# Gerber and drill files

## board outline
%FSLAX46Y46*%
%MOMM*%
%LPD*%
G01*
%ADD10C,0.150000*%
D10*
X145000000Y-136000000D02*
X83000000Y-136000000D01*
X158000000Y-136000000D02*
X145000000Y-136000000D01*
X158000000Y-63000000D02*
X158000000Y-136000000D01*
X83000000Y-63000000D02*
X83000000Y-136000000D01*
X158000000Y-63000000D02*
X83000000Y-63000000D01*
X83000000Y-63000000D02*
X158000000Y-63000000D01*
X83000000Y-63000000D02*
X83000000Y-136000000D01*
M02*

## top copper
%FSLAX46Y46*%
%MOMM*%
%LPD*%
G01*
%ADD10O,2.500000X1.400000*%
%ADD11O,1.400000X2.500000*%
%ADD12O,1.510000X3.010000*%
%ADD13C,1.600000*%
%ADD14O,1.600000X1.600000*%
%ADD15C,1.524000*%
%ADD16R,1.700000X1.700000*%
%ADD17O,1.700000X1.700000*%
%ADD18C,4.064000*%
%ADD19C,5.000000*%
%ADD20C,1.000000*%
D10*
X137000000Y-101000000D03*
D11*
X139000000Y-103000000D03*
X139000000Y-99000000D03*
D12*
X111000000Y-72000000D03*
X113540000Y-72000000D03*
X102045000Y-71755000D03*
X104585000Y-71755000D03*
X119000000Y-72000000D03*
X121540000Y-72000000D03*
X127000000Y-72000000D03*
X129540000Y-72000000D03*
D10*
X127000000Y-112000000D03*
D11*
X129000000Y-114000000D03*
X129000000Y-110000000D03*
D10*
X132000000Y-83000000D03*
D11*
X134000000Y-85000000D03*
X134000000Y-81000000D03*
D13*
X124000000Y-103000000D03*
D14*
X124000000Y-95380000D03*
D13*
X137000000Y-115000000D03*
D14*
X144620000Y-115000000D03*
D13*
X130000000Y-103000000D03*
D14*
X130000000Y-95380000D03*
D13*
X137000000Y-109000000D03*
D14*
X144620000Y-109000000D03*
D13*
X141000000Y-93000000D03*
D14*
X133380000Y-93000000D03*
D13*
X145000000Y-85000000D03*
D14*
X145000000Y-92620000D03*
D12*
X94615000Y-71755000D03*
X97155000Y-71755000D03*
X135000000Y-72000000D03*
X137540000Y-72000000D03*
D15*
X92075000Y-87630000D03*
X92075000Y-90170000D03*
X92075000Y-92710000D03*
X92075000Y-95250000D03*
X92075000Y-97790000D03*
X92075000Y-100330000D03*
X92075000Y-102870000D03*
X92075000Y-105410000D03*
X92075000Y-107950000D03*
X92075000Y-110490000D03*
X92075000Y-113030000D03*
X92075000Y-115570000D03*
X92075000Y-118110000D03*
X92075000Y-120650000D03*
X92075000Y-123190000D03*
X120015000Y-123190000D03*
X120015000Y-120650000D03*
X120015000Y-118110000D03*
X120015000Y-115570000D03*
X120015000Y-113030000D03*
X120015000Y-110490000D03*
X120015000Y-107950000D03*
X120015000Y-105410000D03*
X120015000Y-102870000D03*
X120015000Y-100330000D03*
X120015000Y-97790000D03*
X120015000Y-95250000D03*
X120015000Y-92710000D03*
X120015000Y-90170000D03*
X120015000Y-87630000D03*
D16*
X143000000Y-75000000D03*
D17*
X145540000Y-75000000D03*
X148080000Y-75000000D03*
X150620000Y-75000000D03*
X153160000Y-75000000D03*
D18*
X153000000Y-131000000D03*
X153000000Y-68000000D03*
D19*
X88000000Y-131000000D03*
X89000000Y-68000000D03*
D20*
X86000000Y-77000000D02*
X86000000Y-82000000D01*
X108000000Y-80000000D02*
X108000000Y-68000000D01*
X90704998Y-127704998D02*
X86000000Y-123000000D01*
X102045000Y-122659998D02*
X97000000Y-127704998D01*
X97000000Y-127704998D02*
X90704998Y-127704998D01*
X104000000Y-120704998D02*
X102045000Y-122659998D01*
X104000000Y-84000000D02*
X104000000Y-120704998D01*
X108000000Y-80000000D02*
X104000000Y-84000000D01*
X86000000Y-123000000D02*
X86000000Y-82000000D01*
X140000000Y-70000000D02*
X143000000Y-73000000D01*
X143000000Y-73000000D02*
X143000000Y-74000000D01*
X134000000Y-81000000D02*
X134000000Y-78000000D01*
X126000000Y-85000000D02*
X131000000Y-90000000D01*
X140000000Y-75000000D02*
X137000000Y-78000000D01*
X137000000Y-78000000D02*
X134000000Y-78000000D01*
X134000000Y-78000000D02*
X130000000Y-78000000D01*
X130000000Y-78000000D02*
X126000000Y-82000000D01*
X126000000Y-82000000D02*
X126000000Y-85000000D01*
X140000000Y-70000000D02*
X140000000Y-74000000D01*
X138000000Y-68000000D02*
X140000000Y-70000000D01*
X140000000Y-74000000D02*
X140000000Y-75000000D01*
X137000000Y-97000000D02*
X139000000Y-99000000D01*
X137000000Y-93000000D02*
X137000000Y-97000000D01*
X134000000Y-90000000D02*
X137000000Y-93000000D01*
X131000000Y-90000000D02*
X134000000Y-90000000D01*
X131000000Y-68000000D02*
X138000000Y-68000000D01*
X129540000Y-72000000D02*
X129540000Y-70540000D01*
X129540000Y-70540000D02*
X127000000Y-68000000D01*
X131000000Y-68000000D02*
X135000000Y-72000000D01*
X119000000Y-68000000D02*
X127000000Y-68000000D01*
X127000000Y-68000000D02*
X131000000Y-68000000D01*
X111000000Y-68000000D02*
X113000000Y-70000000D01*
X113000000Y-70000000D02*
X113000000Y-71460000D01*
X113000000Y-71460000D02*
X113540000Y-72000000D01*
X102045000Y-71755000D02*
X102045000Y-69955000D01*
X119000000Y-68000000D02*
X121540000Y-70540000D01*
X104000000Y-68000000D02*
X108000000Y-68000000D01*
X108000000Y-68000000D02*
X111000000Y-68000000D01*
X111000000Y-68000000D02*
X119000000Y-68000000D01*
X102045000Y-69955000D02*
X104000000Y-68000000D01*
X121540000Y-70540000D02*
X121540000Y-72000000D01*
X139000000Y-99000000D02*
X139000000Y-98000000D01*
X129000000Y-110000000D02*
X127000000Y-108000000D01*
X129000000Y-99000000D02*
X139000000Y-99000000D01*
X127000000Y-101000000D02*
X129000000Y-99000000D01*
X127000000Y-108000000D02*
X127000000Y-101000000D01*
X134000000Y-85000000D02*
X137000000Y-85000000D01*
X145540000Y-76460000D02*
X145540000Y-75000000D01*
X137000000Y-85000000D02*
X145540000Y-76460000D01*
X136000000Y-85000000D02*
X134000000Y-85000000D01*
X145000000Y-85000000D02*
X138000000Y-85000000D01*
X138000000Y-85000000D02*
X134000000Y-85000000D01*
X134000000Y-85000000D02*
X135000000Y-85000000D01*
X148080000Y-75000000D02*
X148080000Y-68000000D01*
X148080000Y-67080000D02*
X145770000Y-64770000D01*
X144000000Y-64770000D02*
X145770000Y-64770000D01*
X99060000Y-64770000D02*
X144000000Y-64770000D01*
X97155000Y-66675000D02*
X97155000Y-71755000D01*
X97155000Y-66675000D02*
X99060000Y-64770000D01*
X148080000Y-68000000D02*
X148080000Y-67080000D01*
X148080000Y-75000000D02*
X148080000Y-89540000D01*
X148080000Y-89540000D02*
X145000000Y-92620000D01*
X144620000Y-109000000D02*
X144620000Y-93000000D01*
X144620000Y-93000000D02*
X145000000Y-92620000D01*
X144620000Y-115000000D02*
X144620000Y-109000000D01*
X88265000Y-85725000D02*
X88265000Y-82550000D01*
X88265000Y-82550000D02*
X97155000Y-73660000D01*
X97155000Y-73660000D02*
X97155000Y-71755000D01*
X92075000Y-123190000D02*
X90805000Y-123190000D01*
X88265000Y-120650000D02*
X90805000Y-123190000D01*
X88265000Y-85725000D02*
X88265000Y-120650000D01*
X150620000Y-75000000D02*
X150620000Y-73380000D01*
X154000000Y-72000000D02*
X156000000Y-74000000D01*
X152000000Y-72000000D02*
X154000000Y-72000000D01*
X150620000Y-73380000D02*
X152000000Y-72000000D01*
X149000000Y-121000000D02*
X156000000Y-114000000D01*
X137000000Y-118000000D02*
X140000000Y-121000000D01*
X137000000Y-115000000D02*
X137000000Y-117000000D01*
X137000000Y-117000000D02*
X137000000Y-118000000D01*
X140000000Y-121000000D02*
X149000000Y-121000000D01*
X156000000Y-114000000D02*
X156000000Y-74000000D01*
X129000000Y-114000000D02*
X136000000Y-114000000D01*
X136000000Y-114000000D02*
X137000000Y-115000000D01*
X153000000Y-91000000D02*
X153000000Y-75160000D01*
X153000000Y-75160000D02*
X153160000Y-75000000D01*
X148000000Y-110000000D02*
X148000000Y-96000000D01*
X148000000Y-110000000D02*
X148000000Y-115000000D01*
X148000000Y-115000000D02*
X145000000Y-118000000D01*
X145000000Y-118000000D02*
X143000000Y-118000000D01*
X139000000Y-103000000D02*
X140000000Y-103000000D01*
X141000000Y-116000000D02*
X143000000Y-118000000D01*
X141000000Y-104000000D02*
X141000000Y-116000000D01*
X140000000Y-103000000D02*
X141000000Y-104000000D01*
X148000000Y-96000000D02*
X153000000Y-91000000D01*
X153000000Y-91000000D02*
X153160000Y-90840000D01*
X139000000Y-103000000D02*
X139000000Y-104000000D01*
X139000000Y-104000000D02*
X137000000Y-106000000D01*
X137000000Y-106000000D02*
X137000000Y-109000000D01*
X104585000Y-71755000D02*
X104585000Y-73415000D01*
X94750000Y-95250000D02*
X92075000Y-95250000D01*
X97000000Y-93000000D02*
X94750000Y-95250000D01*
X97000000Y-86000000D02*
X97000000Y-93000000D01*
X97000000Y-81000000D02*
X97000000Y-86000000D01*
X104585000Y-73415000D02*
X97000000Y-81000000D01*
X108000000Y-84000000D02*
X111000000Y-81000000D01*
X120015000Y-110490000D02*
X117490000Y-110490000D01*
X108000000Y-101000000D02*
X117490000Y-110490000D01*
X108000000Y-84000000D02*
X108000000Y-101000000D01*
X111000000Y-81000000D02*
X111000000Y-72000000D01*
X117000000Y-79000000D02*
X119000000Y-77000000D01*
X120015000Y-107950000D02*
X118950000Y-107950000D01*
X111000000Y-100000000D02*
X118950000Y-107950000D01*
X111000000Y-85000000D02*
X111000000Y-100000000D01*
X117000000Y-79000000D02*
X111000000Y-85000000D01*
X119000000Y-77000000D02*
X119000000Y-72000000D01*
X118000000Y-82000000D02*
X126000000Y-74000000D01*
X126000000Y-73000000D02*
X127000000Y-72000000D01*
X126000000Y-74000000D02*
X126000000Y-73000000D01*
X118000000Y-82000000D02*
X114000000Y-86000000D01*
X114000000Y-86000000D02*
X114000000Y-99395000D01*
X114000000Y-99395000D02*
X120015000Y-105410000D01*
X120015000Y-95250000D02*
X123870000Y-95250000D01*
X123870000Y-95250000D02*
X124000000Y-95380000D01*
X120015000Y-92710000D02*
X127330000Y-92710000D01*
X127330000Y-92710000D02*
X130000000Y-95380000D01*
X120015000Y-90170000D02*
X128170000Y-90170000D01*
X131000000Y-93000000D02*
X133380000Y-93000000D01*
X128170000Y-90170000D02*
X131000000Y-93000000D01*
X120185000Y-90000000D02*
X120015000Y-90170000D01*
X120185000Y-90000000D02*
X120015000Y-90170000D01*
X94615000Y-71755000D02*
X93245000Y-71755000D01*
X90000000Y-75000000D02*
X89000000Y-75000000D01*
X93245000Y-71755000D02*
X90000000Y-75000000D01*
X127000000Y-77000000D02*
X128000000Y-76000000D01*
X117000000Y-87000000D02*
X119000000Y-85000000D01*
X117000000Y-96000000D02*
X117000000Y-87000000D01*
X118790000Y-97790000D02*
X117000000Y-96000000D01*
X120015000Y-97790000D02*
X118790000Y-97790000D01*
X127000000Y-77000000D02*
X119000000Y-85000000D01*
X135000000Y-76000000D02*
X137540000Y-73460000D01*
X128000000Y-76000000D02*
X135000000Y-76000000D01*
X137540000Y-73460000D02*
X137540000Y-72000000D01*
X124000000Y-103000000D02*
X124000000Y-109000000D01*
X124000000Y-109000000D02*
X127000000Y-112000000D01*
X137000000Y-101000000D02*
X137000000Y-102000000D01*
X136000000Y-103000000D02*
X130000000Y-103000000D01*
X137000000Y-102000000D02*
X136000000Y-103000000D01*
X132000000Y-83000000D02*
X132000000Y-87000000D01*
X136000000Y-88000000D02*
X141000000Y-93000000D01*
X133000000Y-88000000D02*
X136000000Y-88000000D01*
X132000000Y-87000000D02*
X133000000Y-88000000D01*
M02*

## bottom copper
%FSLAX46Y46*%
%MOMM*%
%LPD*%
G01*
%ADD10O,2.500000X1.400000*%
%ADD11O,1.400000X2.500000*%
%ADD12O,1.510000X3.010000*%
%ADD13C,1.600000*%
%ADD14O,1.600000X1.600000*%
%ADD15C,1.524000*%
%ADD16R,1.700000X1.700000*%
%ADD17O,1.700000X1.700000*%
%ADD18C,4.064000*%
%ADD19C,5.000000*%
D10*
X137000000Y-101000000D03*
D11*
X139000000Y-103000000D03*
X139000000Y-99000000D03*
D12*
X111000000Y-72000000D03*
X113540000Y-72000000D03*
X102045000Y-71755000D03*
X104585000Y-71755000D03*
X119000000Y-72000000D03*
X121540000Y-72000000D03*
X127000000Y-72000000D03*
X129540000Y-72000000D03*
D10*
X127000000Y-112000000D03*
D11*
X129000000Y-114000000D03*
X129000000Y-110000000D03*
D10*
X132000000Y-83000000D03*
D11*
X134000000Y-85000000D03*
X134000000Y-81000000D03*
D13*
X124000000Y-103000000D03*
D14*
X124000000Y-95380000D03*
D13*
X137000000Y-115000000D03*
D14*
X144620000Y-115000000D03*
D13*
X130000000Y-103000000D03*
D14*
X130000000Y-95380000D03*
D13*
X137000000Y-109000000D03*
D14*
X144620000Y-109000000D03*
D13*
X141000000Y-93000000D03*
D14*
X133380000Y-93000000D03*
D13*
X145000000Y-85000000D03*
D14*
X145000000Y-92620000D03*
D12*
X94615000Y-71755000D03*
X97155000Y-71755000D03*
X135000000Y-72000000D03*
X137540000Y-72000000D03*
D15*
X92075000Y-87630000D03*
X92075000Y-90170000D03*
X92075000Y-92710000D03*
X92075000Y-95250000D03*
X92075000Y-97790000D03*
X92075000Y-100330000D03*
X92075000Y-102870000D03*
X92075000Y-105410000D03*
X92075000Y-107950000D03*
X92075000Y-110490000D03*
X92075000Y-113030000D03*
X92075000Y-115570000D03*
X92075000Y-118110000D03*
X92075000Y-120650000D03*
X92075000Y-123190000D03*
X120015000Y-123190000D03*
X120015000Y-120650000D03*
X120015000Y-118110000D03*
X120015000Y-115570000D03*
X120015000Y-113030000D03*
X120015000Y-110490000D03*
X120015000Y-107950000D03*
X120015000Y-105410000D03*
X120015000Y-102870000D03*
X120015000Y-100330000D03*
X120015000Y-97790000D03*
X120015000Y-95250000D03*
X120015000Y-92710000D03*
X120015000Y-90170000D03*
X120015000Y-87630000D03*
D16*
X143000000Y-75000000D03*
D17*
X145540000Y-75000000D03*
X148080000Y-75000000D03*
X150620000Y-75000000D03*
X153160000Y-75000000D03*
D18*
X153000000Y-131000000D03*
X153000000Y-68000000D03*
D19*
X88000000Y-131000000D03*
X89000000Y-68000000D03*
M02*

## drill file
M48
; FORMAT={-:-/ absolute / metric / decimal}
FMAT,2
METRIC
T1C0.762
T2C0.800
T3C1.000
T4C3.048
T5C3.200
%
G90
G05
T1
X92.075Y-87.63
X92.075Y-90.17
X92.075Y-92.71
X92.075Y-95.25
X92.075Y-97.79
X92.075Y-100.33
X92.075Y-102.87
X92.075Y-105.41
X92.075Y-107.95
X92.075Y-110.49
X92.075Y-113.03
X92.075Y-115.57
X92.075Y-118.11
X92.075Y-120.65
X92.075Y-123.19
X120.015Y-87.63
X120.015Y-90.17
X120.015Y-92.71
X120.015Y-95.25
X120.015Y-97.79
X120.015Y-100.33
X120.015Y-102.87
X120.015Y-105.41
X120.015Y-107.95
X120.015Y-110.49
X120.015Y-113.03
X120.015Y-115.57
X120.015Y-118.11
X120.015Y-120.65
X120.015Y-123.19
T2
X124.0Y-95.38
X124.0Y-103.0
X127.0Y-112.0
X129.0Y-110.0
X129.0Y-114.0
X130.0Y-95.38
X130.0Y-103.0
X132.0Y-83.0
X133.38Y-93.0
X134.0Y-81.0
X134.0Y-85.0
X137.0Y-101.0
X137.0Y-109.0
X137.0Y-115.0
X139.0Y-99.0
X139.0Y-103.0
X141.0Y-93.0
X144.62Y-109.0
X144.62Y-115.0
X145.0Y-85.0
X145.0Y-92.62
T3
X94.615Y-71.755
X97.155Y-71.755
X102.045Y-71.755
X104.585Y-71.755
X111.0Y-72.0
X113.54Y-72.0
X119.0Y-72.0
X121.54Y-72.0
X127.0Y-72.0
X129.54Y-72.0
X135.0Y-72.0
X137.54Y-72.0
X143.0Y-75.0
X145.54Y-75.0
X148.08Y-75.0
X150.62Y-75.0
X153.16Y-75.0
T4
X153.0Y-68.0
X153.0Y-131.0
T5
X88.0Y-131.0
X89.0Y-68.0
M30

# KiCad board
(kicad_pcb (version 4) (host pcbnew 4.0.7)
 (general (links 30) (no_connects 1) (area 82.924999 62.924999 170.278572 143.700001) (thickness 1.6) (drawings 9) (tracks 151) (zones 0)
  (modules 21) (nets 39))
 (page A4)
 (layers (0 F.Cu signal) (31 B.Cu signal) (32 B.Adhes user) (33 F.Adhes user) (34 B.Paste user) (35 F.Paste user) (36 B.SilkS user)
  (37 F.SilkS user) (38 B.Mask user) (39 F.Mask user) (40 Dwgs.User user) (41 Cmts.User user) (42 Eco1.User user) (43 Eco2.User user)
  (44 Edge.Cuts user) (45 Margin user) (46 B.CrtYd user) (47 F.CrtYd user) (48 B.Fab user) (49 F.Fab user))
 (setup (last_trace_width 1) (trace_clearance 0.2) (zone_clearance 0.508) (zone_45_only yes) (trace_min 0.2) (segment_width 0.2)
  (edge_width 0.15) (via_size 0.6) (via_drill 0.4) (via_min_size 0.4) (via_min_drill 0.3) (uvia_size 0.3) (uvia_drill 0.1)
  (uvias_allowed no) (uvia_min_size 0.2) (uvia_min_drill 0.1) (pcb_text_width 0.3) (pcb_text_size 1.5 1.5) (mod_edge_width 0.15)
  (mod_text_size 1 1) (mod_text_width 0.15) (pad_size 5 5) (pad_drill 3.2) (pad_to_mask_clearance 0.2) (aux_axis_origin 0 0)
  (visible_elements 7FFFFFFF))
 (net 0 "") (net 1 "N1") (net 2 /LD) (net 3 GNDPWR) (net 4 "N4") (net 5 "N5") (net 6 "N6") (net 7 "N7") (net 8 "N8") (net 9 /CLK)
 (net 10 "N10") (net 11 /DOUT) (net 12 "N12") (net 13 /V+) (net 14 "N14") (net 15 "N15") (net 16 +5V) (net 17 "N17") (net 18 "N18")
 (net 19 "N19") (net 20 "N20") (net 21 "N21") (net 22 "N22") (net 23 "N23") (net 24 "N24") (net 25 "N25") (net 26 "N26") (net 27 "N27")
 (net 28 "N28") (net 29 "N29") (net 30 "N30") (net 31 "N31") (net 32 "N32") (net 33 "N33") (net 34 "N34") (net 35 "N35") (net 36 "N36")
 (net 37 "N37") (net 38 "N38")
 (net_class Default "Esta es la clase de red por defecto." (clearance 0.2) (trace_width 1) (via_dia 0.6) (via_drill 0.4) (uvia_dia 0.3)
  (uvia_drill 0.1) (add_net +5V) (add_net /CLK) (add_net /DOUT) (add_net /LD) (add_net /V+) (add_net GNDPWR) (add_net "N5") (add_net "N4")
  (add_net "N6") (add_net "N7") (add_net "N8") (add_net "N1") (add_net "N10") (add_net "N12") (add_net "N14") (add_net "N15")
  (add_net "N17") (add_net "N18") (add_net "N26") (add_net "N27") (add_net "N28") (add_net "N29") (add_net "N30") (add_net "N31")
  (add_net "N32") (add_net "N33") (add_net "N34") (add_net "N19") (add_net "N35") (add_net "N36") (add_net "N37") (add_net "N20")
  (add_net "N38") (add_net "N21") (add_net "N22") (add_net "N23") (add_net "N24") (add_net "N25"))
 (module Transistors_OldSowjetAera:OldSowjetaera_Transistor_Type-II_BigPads (layer F.Cu) (at 139 101 90)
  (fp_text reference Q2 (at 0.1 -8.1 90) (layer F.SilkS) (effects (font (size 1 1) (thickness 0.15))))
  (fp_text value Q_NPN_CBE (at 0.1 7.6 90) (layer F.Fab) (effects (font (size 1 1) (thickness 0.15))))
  (pad 2 thru_hole oval (at 0 -2 90) (size 1.4 2.5) (drill 0.8) (layers *.Cu *.Mask) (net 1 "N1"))
  (pad 1 thru_hole oval (at -2 0 180) (size 1.4 2.5) (drill 0.8) (layers *.Cu *.Mask) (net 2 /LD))
  (pad 3 thru_hole oval (at 2 0 180) (size 1.4 2.5) (drill 0.8) (layers *.Cu *.Mask) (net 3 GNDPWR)))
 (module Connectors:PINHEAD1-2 (layer F.Cu) (at 111 72)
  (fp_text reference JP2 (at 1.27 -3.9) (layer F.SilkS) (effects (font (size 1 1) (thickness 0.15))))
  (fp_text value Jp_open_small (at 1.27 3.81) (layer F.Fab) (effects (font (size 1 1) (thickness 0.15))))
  (pad 1 thru_hole oval (at 0 0) (size 1.51 3.01) (drill 1) (layers *.Cu *.Mask) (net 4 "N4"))
  (pad 2 thru_hole oval (at 2.54 0) (size 1.51 3.01) (drill 1) (layers *.Cu *.Mask) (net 3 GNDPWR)))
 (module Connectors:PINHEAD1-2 (layer F.Cu) (at 102.045 71.755)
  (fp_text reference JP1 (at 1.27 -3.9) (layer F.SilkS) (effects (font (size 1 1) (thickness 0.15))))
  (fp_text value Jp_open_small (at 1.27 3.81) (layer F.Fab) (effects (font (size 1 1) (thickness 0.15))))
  (pad 1 thru_hole oval (at 0 0) (size 1.51 3.01) (drill 1) (layers *.Cu *.Mask) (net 3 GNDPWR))
  (pad 2 thru_hole oval (at 2.54 0) (size 1.51 3.01) (drill 1) (layers *.Cu *.Mask) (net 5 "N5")))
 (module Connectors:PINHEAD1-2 (layer F.Cu) (at 119 72)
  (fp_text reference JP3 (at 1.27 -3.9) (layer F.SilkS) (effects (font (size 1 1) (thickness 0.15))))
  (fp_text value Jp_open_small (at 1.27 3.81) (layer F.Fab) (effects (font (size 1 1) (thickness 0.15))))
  (pad 1 thru_hole oval (at 0 0) (size 1.51 3.01) (drill 1) (layers *.Cu *.Mask) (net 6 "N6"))
  (pad 2 thru_hole oval (at 2.54 0) (size 1.51 3.01) (drill 1) (layers *.Cu *.Mask) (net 3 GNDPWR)))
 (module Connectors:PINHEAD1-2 (layer F.Cu) (at 127 72)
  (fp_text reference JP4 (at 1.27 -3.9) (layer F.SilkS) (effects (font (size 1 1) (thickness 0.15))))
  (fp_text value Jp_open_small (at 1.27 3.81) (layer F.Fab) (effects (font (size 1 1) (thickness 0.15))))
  (pad 1 thru_hole oval (at 0 0) (size 1.51 3.01) (drill 1) (layers *.Cu *.Mask) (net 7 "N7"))
  (pad 2 thru_hole oval (at 2.54 0) (size 1.51 3.01) (drill 1) (layers *.Cu *.Mask) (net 3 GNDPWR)))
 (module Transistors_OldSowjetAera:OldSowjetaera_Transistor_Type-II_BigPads (layer F.Cu) (at 129 112 90)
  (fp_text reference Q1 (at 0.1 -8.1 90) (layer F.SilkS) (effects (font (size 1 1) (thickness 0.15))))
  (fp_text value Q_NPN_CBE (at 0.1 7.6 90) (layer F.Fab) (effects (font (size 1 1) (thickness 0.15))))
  (pad 2 thru_hole oval (at 0 -2 90) (size 1.4 2.5) (drill 0.8) (layers *.Cu *.Mask) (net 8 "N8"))
  (pad 1 thru_hole oval (at -2 0 180) (size 1.4 2.5) (drill 0.8) (layers *.Cu *.Mask) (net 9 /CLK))
  (pad 3 thru_hole oval (at 2 0 180) (size 1.4 2.5) (drill 0.8) (layers *.Cu *.Mask) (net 3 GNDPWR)))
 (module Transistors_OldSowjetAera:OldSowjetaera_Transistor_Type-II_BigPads (layer F.Cu) (at 134 83 90)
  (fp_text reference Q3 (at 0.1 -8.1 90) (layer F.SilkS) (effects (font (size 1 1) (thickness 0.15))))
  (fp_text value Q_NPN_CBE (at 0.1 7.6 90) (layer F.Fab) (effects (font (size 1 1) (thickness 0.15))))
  (pad 2 thru_hole oval (at 0 -2 90) (size 1.4 2.5) (drill 0.8) (layers *.Cu *.Mask) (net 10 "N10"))
  (pad 1 thru_hole oval (at -2 0 180) (size 1.4 2.5) (drill 0.8) (layers *.Cu *.Mask) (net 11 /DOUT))
  (pad 3 thru_hole oval (at 2 0 180) (size 1.4 2.5) (drill 0.8) (layers *.Cu *.Mask) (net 3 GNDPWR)))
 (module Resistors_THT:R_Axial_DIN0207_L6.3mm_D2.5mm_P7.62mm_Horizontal (layer F.Cu) (at 124 103 90)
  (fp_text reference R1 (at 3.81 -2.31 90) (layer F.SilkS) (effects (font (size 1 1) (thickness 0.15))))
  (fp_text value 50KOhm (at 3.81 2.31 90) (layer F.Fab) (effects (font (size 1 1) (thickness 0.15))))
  (pad 1 thru_hole circle (at 0 0 90) (size 1.6 1.6) (drill 0.8) (layers *.Cu *.Mask) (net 8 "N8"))
  (pad 2 thru_hole oval (at 7.62 0 90) (size 1.6 1.6) (drill 0.8) (layers *.Cu *.Mask) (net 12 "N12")))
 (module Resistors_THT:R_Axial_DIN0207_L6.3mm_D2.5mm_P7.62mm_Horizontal (layer F.Cu) (at 137 115)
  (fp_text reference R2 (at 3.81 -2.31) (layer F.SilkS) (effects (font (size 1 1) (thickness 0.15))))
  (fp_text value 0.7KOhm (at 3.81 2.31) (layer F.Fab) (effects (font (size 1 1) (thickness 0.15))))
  (pad 1 thru_hole circle (at 0 0) (size 1.6 1.6) (drill 0.8) (layers *.Cu *.Mask) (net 9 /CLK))
  (pad 2 thru_hole oval (at 7.62 0) (size 1.6 1.6) (drill 0.8) (layers *.Cu *.Mask) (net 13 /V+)))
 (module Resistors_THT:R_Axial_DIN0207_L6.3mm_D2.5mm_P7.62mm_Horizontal (layer F.Cu) (at 130 103 90)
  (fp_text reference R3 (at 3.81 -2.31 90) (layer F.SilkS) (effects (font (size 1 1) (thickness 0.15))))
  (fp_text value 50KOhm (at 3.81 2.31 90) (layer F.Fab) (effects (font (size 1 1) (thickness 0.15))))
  (pad 1 thru_hole circle (at 0 0 90) (size 1.6 1.6) (drill 0.8) (layers *.Cu *.Mask) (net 1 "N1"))
  (pad 2 thru_hole oval (at 7.62 0 90) (size 1.6 1.6) (drill 0.8) (layers *.Cu *.Mask) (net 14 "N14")))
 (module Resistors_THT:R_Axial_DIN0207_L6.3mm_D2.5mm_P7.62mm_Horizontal (layer F.Cu) (at 137 109)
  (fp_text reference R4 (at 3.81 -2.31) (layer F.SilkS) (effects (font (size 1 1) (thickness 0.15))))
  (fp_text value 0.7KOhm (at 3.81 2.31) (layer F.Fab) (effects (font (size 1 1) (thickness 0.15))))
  (pad 1 thru_hole circle (at 0 0) (size 1.6 1.6) (drill 0.8) (layers *.Cu *.Mask) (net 2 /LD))
  (pad 2 thru_hole oval (at 7.62 0) (size 1.6 1.6) (drill 0.8) (layers *.Cu *.Mask) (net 13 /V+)))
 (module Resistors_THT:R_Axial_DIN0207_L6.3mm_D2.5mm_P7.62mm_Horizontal (layer F.Cu) (at 141 93 180)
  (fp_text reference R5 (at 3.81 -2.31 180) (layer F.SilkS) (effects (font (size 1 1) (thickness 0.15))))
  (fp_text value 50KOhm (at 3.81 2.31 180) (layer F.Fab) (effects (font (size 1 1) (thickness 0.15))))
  (pad 1 thru_hole circle (at 0 0 180) (size 1.6 1.6) (drill 0.8) (layers *.Cu *.Mask) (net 10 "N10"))
  (pad 2 thru_hole oval (at 7.62 0 180) (size 1.6 1.6) (drill 0.8) (layers *.Cu *.Mask) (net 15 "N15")))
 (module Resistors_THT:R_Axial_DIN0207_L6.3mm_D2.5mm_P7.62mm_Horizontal (layer F.Cu) (at 145 85 270)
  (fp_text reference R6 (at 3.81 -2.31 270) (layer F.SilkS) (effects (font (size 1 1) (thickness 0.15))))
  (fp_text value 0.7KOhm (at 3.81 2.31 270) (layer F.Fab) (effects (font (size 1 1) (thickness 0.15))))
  (pad 1 thru_hole circle (at 0 0 270) (size 1.6 1.6) (drill 0.8) (layers *.Cu *.Mask) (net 11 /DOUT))
  (pad 2 thru_hole oval (at 7.62 0 270) (size 1.6 1.6) (drill 0.8) (layers *.Cu *.Mask) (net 13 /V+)))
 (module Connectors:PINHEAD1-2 (layer F.Cu) (at 94.615 71.755)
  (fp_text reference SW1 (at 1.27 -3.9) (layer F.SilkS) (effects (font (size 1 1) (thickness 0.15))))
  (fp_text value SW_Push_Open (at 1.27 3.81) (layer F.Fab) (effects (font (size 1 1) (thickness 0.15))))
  (pad 1 thru_hole oval (at 0 0) (size 1.51 3.01) (drill 1) (layers *.Cu *.Mask) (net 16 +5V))
  (pad 2 thru_hole oval (at 2.54 0) (size 1.51 3.01) (drill 1) (layers *.Cu *.Mask) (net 13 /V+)))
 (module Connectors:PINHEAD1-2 (layer F.Cu) (at 135 72)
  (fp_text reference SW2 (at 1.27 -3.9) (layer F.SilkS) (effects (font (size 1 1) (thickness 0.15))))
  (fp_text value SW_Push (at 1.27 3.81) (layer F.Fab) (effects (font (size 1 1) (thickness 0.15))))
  (pad 1 thru_hole oval (at 0 0) (size 1.51 3.01) (drill 1) (layers *.Cu *.Mask) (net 3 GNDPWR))
  (pad 2 thru_hole oval (at 2.54 0) (size 1.51 3.01) (drill 1) (layers *.Cu *.Mask) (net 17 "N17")))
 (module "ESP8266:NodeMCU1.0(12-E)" (layer F.Cu) (at 106.045 107.95)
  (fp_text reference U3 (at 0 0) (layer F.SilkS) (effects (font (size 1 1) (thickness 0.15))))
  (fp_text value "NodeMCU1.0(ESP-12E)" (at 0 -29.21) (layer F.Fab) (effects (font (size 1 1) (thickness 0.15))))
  (pad 1 thru_hole circle (at -13.97 -20.32) (size 1.524 1.524) (drill 0.762) (layers *.Cu *.Mask F.SilkS) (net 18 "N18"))
  (pad 2 thru_hole circle (at -13.97 -17.78) (size 1.524 1.524) (drill 0.762) (layers *.Cu *.Mask F.SilkS) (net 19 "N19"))
  (pad 3 thru_hole circle (at -13.97 -15.24) (size 1.524 1.524) (drill 0.762) (layers *.Cu *.Mask F.SilkS) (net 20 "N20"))
  (pad 4 thru_hole circle (at -13.97 -12.7) (size 1.524 1.524) (drill 0.762) (layers *.Cu *.Mask F.SilkS) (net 5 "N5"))
  (pad 5 thru_hole circle (at -13.97 -10.16) (size 1.524 1.524) (drill 0.762) (layers *.Cu *.Mask F.SilkS) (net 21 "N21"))
  (pad 6 thru_hole circle (at -13.97 -7.62) (size 1.524 1.524) (drill 0.762) (layers *.Cu *.Mask F.SilkS) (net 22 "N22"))
  (pad 7 thru_hole circle (at -13.97 -5.08) (size 1.524 1.524) (drill 0.762) (layers *.Cu *.Mask F.SilkS) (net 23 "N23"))
  (pad 8 thru_hole circle (at -13.97 -2.54) (size 1.524 1.524) (drill 0.762) (layers *.Cu *.Mask F.SilkS) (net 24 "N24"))
  (pad 9 thru_hole circle (at -13.97 0) (size 1.524 1.524) (drill 0.762) (layers *.Cu *.Mask F.SilkS) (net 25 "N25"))
  (pad 10 thru_hole circle (at -13.97 2.54) (size 1.524 1.524) (drill 0.762) (layers *.Cu *.Mask F.SilkS) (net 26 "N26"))
  (pad 11 thru_hole circle (at -13.97 5.08) (size 1.524 1.524) (drill 0.762) (layers *.Cu *.Mask F.SilkS) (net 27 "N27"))
  (pad 12 thru_hole circle (at -13.97 7.62) (size 1.524 1.524) (drill 0.762) (layers *.Cu *.Mask F.SilkS) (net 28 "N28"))
  (pad 13 thru_hole circle (at -13.97 10.16) (size 1.524 1.524) (drill 0.762) (layers *.Cu *.Mask F.SilkS) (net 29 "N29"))
  (pad 14 thru_hole circle (at -13.97 12.7) (size 1.524 1.524) (drill 0.762) (layers *.Cu *.Mask F.SilkS) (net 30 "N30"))
  (pad 15 thru_hole circle (at -13.97 15.24) (size 1.524 1.524) (drill 0.762) (layers *.Cu *.Mask F.SilkS) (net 13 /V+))
  (pad 16 thru_hole circle (at 13.97 15.24) (size 1.524 1.524) (drill 0.762) (layers *.Cu *.Mask F.SilkS) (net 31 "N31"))
  (pad 17 thru_hole circle (at 13.97 12.7) (size 1.524 1.524) (drill 0.762) (layers *.Cu *.Mask F.SilkS) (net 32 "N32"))
  (pad 18 thru_hole circle (at 13.97 10.16) (size 1.524 1.524) (drill 0.762) (layers *.Cu *.Mask F.SilkS) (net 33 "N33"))
  (pad 19 thru_hole circle (at 13.97 7.62) (size 1.524 1.524) (drill 0.762) (layers *.Cu *.Mask F.SilkS) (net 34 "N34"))
  (pad 20 thru_hole circle (at 13.97 5.08) (size 1.524 1.524) (drill 0.762) (layers *.Cu *.Mask F.SilkS) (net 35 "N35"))
  (pad 21 thru_hole circle (at 13.97 2.54) (size 1.524 1.524) (drill 0.762) (layers *.Cu *.Mask F.SilkS) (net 4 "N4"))
  (pad 22 thru_hole circle (at 13.97 0) (size 1.524 1.524) (drill 0.762) (layers *.Cu *.Mask F.SilkS) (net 6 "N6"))
  (pad 23 thru_hole circle (at 13.97 -2.54) (size 1.524 1.524) (drill 0.762) (layers *.Cu *.Mask F.SilkS) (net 7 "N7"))
  (pad 24 thru_hole circle (at 13.97 -5.08) (size 1.524 1.524) (drill 0.762) (layers *.Cu *.Mask F.SilkS) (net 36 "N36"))
  (pad 25 thru_hole circle (at 13.97 -7.62) (size 1.524 1.524) (drill 0.762) (layers *.Cu *.Mask F.SilkS) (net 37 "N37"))
  (pad 26 thru_hole circle (at 13.97 -10.16) (size 1.524 1.524) (drill 0.762) (layers *.Cu *.Mask F.SilkS) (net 17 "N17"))
  (pad 27 thru_hole circle (at 13.97 -12.7) (size 1.524 1.524) (drill 0.762) (layers *.Cu *.Mask F.SilkS) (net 12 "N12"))
  (pad 28 thru_hole circle (at 13.97 -15.24) (size 1.524 1.524) (drill 0.762) (layers *.Cu *.Mask F.SilkS) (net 14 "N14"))
  (pad 29 thru_hole circle (at 13.97 -17.78) (size 1.524 1.524) (drill 0.762) (layers *.Cu *.Mask F.SilkS) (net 15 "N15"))
  (pad 30 thru_hole circle (at 13.97 -20.32) (size 1.524 1.524) (drill 0.762) (layers *.Cu *.Mask F.SilkS) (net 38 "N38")))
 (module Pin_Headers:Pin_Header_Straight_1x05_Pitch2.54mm (layer F.Cu) (at 143 75 90)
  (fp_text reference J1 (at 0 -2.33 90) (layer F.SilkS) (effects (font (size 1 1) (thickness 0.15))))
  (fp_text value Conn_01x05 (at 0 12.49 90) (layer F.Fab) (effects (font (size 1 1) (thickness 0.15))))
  (pad 1 thru_hole rect (at 0 0 90) (size 1.7 1.7) (drill 1) (layers *.Cu *.Mask) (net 3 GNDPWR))
  (pad 2 thru_hole oval (at 0 2.54 90) (size 1.7 1.7) (drill 1) (layers *.Cu *.Mask) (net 11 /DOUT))
  (pad 3 thru_hole oval (at 0 5.08 90) (size 1.7 1.7) (drill 1) (layers *.Cu *.Mask) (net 13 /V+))
  (pad 4 thru_hole oval (at 0 7.62 90) (size 1.7 1.7) (drill 1) (layers *.Cu *.Mask) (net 9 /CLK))
  (pad 5 thru_hole oval (at 0 10.16 90) (size 1.7 1.7) (drill 1) (layers *.Cu *.Mask) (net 2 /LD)))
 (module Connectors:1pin (layer F.Cu) (at 153 131)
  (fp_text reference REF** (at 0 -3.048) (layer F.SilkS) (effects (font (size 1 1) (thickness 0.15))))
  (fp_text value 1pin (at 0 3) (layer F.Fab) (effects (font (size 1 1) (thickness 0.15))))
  (pad 1 thru_hole circle (at 0 0) (size 4.064 4.064) (drill 3.048) (layers *.Cu *.Mask)))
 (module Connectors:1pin (layer F.Cu) (at 153 68)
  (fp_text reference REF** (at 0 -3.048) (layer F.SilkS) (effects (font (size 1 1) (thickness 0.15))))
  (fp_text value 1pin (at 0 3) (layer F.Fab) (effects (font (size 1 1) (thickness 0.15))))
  (pad 1 thru_hole circle (at 0 0) (size 4.064 4.064) (drill 3.048) (layers *.Cu *.Mask)))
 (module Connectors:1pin (layer F.Cu) (at 88 131)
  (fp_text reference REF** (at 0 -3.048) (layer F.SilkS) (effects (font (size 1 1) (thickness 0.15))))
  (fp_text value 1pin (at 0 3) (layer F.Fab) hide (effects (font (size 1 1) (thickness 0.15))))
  (pad 1 thru_hole circle (at 0 0) (size 5 5) (drill 3.2) (layers *.Cu *.Mask)))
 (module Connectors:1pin (layer F.Cu) (at 89 68)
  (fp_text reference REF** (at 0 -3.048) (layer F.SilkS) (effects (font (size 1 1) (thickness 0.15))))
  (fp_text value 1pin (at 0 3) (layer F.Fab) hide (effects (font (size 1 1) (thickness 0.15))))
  (pad 1 thru_hole circle (at 0 0) (size 5 5) (drill 3.2) (layers *.Cu *.Mask)))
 (gr_line (start 145 136) (end 83 136) (angle 90) (layer Edge.Cuts) (width 0.15))
 (gr_line (start 158 136) (end 145 136) (angle 90) (layer Edge.Cuts) (width 0.15))
 (gr_line (start 158 63) (end 158 136) (angle 90) (layer Edge.Cuts) (width 0.15))
 (gr_line (start 83 63) (end 83 136) (angle 90) (layer Edge.Cuts) (width 0.15))
 (gr_line (start 158 63) (end 83 63) (angle 90) (layer Edge.Cuts) (width 0.15))
 (gr_line (start 83 63) (end 158 63) (angle 90) (layer Edge.Cuts) (width 0.15))
 (gr_line (start 83 63) (end 83 136) (angle 90) (layer Edge.Cuts) (width 0.15))
 (segment (start 86 77) (end 86 82) (width 1) (layer F.Cu) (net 3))
 (segment (start 108 80) (end 108 68) (width 1) (layer F.Cu) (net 3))
 (segment (start 90.704998 127.704998) (end 86 123) (width 1) (layer F.Cu) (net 3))
 (segment (start 102.045 122.659998) (end 97 127.704998) (width 1) (layer F.Cu) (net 3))
 (segment (start 97 127.704998) (end 90.704998 127.704998) (width 1) (layer F.Cu) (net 3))
 (segment (start 104 120.704998) (end 102.045 122.659998) (width 1) (layer F.Cu) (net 3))
 (segment (start 104 84) (end 104 120.704998) (width 1) (layer F.Cu) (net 3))
 (segment (start 108 80) (end 104 84) (width 1) (layer F.Cu) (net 3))
 (segment (start 86 123) (end 86 82) (width 1) (layer F.Cu) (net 3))
 (segment (start 140 70) (end 143 73) (width 1) (layer F.Cu) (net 3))
 (segment (start 143 73) (end 143 74) (width 1) (layer F.Cu) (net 3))
 (segment (start 134 81) (end 134 78) (width 1) (layer F.Cu) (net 3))
 (segment (start 126 85) (end 131 90) (width 1) (layer F.Cu) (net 3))
 (segment (start 140 75) (end 137 78) (width 1) (layer F.Cu) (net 3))
 (segment (start 137 78) (end 134 78) (width 1) (layer F.Cu) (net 3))
 (segment (start 134 78) (end 130 78) (width 1) (layer F.Cu) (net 3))
 (segment (start 130 78) (end 126 82) (width 1) (layer F.Cu) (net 3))
 (segment (start 126 82) (end 126 85) (width 1) (layer F.Cu) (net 3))
 (segment (start 140 70) (end 140 74) (width 1) (layer F.Cu) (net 3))
 (segment (start 138 68) (end 140 70) (width 1) (layer F.Cu) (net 3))
 (segment (start 140 74) (end 140 75) (width 1) (layer F.Cu) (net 3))
 (segment (start 137 97) (end 139 99) (width 1) (layer F.Cu) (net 3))
 (segment (start 137 93) (end 137 97) (width 1) (layer F.Cu) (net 3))
 (segment (start 134 90) (end 137 93) (width 1) (layer F.Cu) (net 3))
 (segment (start 131 90) (end 134 90) (width 1) (layer F.Cu) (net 3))
 (segment (start 131 68) (end 138 68) (width 1) (layer F.Cu) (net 3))
 (segment (start 129.54 72) (end 129.54 70.54) (width 1) (layer F.Cu) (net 3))
 (segment (start 129.54 70.54) (end 127 68) (width 1) (layer F.Cu) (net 3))
 (segment (start 131 68) (end 135 72) (width 1) (layer F.Cu) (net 3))
 (segment (start 119 68) (end 127 68) (width 1) (layer F.Cu) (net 3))
 (segment (start 127 68) (end 131 68) (width 1) (layer F.Cu) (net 3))
 (segment (start 111 68) (end 113 70) (width 1) (layer F.Cu) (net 3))
 (segment (start 113 70) (end 113 71.46) (width 1) (layer F.Cu) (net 3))
 (segment (start 113 71.46) (end 113.54 72) (width 1) (layer F.Cu) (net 3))
 (segment (start 102.045 71.755) (end 102.045 69.955) (width 1) (layer F.Cu) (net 3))
 (segment (start 119 68) (end 121.54 70.54) (width 1) (layer F.Cu) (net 3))
 (segment (start 104 68) (end 108 68) (width 1) (layer F.Cu) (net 3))
 (segment (start 108 68) (end 111 68) (width 1) (layer F.Cu) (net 3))
 (segment (start 111 68) (end 119 68) (width 1) (layer F.Cu) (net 3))
 (segment (start 102.045 69.955) (end 104 68) (width 1) (layer F.Cu) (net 3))
 (segment (start 121.54 70.54) (end 121.54 72) (width 1) (layer F.Cu) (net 3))
 (segment (start 139 99) (end 139 98) (width 1) (layer F.Cu) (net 3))
 (segment (start 129 110) (end 127 108) (width 1) (layer F.Cu) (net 3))
 (segment (start 129 99) (end 139 99) (width 1) (layer F.Cu) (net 3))
 (segment (start 127 101) (end 129 99) (width 1) (layer F.Cu) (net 3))
 (segment (start 127 108) (end 127 101) (width 1) (layer F.Cu) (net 3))
 (segment (start 134 85) (end 137 85) (width 1) (layer F.Cu) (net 11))
 (segment (start 145.54 76.46) (end 145.54 75) (width 1) (layer F.Cu) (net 11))
 (segment (start 137 85) (end 145.54 76.46) (width 1) (layer F.Cu) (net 11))
 (segment (start 136 85) (end 134 85) (width 1) (layer F.Cu) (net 11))
 (segment (start 145 85) (end 138 85) (width 1) (layer F.Cu) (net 11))
 (segment (start 138 85) (end 134 85) (width 1) (layer F.Cu) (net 11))
 (segment (start 134 85) (end 135 85) (width 1) (layer F.Cu) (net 11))
 (segment (start 148.08 75) (end 148.08 68) (width 1) (layer F.Cu) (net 13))
 (segment (start 148.08 67.08) (end 145.77 64.77) (width 1) (layer F.Cu) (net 13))
 (segment (start 144 64.77) (end 145.77 64.77) (width 1) (layer F.Cu) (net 13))
 (segment (start 99.06 64.77) (end 144 64.77) (width 1) (layer F.Cu) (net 13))
 (segment (start 97.155 66.675) (end 97.155 71.755) (width 1) (layer F.Cu) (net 13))
 (segment (start 97.155 66.675) (end 99.06 64.77) (width 1) (layer F.Cu) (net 13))
 (segment (start 148.08 68) (end 148.08 67.08) (width 1) (layer F.Cu) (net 13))
 (segment (start 148.08 75) (end 148.08 89.54) (width 1) (layer F.Cu) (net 13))
 (segment (start 148.08 89.54) (end 145 92.62) (width 1) (layer F.Cu) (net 13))
 (segment (start 144.62 109) (end 144.62 93) (width 1) (layer F.Cu) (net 13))
 (segment (start 144.62 93) (end 145 92.62) (width 1) (layer F.Cu) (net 13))
 (segment (start 144.62 115) (end 144.62 109) (width 1) (layer F.Cu) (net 13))
 (segment (start 88.265 85.725) (end 88.265 82.55) (width 1) (layer F.Cu) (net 13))
 (segment (start 88.265 82.55) (end 97.155 73.66) (width 1) (layer F.Cu) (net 13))
 (segment (start 97.155 73.66) (end 97.155 71.755) (width 1) (layer F.Cu) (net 13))
 (segment (start 92.075 123.19) (end 90.805 123.19) (width 1) (layer F.Cu) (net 13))
 (segment (start 88.265 120.65) (end 90.805 123.19) (width 1) (layer F.Cu) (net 13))
 (segment (start 88.265 85.725) (end 88.265 120.65) (width 1) (layer F.Cu) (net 13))
 (segment (start 150.62 75) (end 150.62 73.38) (width 1) (layer F.Cu) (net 9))
 (segment (start 154 72) (end 156 74) (width 1) (layer F.Cu) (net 9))
 (segment (start 152 72) (end 154 72) (width 1) (layer F.Cu) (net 9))
 (segment (start 150.62 73.38) (end 152 72) (width 1) (layer F.Cu) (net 9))
 (segment (start 149 121) (end 156 114) (width 1) (layer F.Cu) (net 9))
 (segment (start 137 118) (end 140 121) (width 1) (layer F.Cu) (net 9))
 (segment (start 137 115) (end 137 117) (width 1) (layer F.Cu) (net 9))
 (segment (start 137 117) (end 137 118) (width 1) (layer F.Cu) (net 9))
 (segment (start 140 121) (end 149 121) (width 1) (layer F.Cu) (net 9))
 (segment (start 156 114) (end 156 74) (width 1) (layer F.Cu) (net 9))
 (segment (start 129 114) (end 136 114) (width 1) (layer F.Cu) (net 9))
 (segment (start 136 114) (end 137 115) (width 1) (layer F.Cu) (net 9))
 (segment (start 153 91) (end 153 75.16) (width 1) (layer F.Cu) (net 2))
 (segment (start 153 75.16) (end 153.16 75) (width 1) (layer F.Cu) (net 2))
 (segment (start 148 110) (end 148 96) (width 1) (layer F.Cu) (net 2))
 (segment (start 148 110) (end 148 115) (width 1) (layer F.Cu) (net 2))
 (segment (start 148 115) (end 145 118) (width 1) (layer F.Cu) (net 2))
 (segment (start 145 118) (end 143 118) (width 1) (layer F.Cu) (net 2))
 (segment (start 139 103) (end 140 103) (width 1) (layer F.Cu) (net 2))
 (segment (start 141 116) (end 143 118) (width 1) (layer F.Cu) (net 2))
 (segment (start 141 104) (end 141 116) (width 1) (layer F.Cu) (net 2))
 (segment (start 140 103) (end 141 104) (width 1) (layer F.Cu) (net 2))
 (segment (start 148 96) (end 153 91) (width 1) (layer F.Cu) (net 2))
 (segment (start 153 91) (end 153.16 90.84) (width 1) (layer F.Cu) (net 2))
 (segment (start 139 103) (end 139 104) (width 1) (layer F.Cu) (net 2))
 (segment (start 139 104) (end 137 106) (width 1) (layer F.Cu) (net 2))
 (segment (start 137 106) (end 137 109) (width 1) (layer F.Cu) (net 2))
 (segment (start 104.585 71.755) (end 104.585 73.415) (width 1) (layer F.Cu) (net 5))
 (segment (start 94.75 95.25) (end 92.075 95.25) (width 1) (layer F.Cu) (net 5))
 (segment (start 97 93) (end 94.75 95.25) (width 1) (layer F.Cu) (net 5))
 (segment (start 97 86) (end 97 93) (width 1) (layer F.Cu) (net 5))
 (segment (start 97 81) (end 97 86) (width 1) (layer F.Cu) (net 5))
 (segment (start 104.585 73.415) (end 97 81) (width 1) (layer F.Cu) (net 5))
 (segment (start 108 84) (end 111 81) (width 1) (layer F.Cu) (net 4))
 (segment (start 120.015 110.49) (end 117.49 110.49) (width 1) (layer F.Cu) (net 4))
 (segment (start 108 101) (end 117.49 110.49) (width 1) (layer F.Cu) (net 4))
 (segment (start 108 84) (end 108 101) (width 1) (layer F.Cu) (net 4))
 (segment (start 111 81) (end 111 72) (width 1) (layer F.Cu) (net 4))
 (segment (start 117 79) (end 119 77) (width 1) (layer F.Cu) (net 6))
 (segment (start 120.015 107.95) (end 118.95 107.95) (width 1) (layer F.Cu) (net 6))
 (segment (start 111 100) (end 118.95 107.95) (width 1) (layer F.Cu) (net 6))
 (segment (start 111 85) (end 111 100) (width 1) (layer F.Cu) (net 6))
 (segment (start 117 79) (end 111 85) (width 1) (layer F.Cu) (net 6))
 (segment (start 119 77) (end 119 72) (width 1) (layer F.Cu) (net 6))
 (segment (start 118 82) (end 126 74) (width 1) (layer F.Cu) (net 7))
 (segment (start 126 73) (end 127 72) (width 1) (layer F.Cu) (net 7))
 (segment (start 126 74) (end 126 73) (width 1) (layer F.Cu) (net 7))
 (segment (start 118 82) (end 114 86) (width 1) (layer F.Cu) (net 7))
 (segment (start 114 86) (end 114 99.395) (width 1) (layer F.Cu) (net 7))
 (segment (start 114 99.395) (end 120.015 105.41) (width 1) (layer F.Cu) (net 7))
 (segment (start 120.015 95.25) (end 123.87 95.25) (width 1) (layer F.Cu) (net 12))
 (segment (start 123.87 95.25) (end 124 95.38) (width 1) (layer F.Cu) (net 12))
 (segment (start 120.015 92.71) (end 127.33 92.71) (width 1) (layer F.Cu) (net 14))
 (segment (start 127.33 92.71) (end 130 95.38) (width 1) (layer F.Cu) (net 14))
 (segment (start 120.015 90.17) (end 128.17 90.17) (width 1) (layer F.Cu) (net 15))
 (segment (start 131 93) (end 133.38 93) (width 1) (layer F.Cu) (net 15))
 (segment (start 128.17 90.17) (end 131 93) (width 1) (layer F.Cu) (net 15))
 (segment (start 120.185 90) (end 120.015 90.17) (width 1) (layer F.Cu) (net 15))
 (segment (start 120.185 90) (end 120.015 90.17) (width 1) (layer F.Cu) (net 15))
 (segment (start 94.615 71.755) (end 93.245 71.755) (width 1) (layer F.Cu) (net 16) (status 400000))
 (segment (start 90 75) (end 89 75) (width 1) (layer F.Cu) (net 16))
 (segment (start 93.245 71.755) (end 90 75) (width 1) (layer F.Cu) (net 16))
 (segment (start 127 77) (end 128 76) (width 1) (layer F.Cu) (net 17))
 (segment (start 117 87) (end 119 85) (width 1) (layer F.Cu) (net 17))
 (segment (start 117 96) (end 117 87) (width 1) (layer F.Cu) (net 17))
 (segment (start 118.79 97.79) (end 117 96) (width 1) (layer F.Cu) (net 17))
 (segment (start 120.015 97.79) (end 118.79 97.79) (width 1) (layer F.Cu) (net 17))
 (segment (start 127 77) (end 119 85) (width 1) (layer F.Cu) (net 17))
 (segment (start 135 76) (end 137.54 73.46) (width 1) (layer F.Cu) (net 17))
 (segment (start 128 76) (end 135 76) (width 1) (layer F.Cu) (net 17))
 (segment (start 137.54 73.46) (end 137.54 72) (width 1) (layer F.Cu) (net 17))
 (segment (start 124 103) (end 124 109) (width 1) (layer F.Cu) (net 8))
 (segment (start 124 109) (end 127 112) (width 1) (layer F.Cu) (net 8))
 (segment (start 137 101) (end 137 102) (width 1) (layer F.Cu) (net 1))
 (segment (start 136 103) (end 130 103) (width 1) (layer F.Cu) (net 1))
 (segment (start 137 102) (end 136 103) (width 1) (layer F.Cu) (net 1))
 (segment (start 132 83) (end 132 87) (width 1) (layer F.Cu) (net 10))
 (segment (start 136 88) (end 141 93) (width 1) (layer F.Cu) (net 10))
 (segment (start 133 88) (end 136 88) (width 1) (layer F.Cu) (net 10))
 (segment (start 132 87) (end 133 88) (width 1) (layer F.Cu) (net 10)))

